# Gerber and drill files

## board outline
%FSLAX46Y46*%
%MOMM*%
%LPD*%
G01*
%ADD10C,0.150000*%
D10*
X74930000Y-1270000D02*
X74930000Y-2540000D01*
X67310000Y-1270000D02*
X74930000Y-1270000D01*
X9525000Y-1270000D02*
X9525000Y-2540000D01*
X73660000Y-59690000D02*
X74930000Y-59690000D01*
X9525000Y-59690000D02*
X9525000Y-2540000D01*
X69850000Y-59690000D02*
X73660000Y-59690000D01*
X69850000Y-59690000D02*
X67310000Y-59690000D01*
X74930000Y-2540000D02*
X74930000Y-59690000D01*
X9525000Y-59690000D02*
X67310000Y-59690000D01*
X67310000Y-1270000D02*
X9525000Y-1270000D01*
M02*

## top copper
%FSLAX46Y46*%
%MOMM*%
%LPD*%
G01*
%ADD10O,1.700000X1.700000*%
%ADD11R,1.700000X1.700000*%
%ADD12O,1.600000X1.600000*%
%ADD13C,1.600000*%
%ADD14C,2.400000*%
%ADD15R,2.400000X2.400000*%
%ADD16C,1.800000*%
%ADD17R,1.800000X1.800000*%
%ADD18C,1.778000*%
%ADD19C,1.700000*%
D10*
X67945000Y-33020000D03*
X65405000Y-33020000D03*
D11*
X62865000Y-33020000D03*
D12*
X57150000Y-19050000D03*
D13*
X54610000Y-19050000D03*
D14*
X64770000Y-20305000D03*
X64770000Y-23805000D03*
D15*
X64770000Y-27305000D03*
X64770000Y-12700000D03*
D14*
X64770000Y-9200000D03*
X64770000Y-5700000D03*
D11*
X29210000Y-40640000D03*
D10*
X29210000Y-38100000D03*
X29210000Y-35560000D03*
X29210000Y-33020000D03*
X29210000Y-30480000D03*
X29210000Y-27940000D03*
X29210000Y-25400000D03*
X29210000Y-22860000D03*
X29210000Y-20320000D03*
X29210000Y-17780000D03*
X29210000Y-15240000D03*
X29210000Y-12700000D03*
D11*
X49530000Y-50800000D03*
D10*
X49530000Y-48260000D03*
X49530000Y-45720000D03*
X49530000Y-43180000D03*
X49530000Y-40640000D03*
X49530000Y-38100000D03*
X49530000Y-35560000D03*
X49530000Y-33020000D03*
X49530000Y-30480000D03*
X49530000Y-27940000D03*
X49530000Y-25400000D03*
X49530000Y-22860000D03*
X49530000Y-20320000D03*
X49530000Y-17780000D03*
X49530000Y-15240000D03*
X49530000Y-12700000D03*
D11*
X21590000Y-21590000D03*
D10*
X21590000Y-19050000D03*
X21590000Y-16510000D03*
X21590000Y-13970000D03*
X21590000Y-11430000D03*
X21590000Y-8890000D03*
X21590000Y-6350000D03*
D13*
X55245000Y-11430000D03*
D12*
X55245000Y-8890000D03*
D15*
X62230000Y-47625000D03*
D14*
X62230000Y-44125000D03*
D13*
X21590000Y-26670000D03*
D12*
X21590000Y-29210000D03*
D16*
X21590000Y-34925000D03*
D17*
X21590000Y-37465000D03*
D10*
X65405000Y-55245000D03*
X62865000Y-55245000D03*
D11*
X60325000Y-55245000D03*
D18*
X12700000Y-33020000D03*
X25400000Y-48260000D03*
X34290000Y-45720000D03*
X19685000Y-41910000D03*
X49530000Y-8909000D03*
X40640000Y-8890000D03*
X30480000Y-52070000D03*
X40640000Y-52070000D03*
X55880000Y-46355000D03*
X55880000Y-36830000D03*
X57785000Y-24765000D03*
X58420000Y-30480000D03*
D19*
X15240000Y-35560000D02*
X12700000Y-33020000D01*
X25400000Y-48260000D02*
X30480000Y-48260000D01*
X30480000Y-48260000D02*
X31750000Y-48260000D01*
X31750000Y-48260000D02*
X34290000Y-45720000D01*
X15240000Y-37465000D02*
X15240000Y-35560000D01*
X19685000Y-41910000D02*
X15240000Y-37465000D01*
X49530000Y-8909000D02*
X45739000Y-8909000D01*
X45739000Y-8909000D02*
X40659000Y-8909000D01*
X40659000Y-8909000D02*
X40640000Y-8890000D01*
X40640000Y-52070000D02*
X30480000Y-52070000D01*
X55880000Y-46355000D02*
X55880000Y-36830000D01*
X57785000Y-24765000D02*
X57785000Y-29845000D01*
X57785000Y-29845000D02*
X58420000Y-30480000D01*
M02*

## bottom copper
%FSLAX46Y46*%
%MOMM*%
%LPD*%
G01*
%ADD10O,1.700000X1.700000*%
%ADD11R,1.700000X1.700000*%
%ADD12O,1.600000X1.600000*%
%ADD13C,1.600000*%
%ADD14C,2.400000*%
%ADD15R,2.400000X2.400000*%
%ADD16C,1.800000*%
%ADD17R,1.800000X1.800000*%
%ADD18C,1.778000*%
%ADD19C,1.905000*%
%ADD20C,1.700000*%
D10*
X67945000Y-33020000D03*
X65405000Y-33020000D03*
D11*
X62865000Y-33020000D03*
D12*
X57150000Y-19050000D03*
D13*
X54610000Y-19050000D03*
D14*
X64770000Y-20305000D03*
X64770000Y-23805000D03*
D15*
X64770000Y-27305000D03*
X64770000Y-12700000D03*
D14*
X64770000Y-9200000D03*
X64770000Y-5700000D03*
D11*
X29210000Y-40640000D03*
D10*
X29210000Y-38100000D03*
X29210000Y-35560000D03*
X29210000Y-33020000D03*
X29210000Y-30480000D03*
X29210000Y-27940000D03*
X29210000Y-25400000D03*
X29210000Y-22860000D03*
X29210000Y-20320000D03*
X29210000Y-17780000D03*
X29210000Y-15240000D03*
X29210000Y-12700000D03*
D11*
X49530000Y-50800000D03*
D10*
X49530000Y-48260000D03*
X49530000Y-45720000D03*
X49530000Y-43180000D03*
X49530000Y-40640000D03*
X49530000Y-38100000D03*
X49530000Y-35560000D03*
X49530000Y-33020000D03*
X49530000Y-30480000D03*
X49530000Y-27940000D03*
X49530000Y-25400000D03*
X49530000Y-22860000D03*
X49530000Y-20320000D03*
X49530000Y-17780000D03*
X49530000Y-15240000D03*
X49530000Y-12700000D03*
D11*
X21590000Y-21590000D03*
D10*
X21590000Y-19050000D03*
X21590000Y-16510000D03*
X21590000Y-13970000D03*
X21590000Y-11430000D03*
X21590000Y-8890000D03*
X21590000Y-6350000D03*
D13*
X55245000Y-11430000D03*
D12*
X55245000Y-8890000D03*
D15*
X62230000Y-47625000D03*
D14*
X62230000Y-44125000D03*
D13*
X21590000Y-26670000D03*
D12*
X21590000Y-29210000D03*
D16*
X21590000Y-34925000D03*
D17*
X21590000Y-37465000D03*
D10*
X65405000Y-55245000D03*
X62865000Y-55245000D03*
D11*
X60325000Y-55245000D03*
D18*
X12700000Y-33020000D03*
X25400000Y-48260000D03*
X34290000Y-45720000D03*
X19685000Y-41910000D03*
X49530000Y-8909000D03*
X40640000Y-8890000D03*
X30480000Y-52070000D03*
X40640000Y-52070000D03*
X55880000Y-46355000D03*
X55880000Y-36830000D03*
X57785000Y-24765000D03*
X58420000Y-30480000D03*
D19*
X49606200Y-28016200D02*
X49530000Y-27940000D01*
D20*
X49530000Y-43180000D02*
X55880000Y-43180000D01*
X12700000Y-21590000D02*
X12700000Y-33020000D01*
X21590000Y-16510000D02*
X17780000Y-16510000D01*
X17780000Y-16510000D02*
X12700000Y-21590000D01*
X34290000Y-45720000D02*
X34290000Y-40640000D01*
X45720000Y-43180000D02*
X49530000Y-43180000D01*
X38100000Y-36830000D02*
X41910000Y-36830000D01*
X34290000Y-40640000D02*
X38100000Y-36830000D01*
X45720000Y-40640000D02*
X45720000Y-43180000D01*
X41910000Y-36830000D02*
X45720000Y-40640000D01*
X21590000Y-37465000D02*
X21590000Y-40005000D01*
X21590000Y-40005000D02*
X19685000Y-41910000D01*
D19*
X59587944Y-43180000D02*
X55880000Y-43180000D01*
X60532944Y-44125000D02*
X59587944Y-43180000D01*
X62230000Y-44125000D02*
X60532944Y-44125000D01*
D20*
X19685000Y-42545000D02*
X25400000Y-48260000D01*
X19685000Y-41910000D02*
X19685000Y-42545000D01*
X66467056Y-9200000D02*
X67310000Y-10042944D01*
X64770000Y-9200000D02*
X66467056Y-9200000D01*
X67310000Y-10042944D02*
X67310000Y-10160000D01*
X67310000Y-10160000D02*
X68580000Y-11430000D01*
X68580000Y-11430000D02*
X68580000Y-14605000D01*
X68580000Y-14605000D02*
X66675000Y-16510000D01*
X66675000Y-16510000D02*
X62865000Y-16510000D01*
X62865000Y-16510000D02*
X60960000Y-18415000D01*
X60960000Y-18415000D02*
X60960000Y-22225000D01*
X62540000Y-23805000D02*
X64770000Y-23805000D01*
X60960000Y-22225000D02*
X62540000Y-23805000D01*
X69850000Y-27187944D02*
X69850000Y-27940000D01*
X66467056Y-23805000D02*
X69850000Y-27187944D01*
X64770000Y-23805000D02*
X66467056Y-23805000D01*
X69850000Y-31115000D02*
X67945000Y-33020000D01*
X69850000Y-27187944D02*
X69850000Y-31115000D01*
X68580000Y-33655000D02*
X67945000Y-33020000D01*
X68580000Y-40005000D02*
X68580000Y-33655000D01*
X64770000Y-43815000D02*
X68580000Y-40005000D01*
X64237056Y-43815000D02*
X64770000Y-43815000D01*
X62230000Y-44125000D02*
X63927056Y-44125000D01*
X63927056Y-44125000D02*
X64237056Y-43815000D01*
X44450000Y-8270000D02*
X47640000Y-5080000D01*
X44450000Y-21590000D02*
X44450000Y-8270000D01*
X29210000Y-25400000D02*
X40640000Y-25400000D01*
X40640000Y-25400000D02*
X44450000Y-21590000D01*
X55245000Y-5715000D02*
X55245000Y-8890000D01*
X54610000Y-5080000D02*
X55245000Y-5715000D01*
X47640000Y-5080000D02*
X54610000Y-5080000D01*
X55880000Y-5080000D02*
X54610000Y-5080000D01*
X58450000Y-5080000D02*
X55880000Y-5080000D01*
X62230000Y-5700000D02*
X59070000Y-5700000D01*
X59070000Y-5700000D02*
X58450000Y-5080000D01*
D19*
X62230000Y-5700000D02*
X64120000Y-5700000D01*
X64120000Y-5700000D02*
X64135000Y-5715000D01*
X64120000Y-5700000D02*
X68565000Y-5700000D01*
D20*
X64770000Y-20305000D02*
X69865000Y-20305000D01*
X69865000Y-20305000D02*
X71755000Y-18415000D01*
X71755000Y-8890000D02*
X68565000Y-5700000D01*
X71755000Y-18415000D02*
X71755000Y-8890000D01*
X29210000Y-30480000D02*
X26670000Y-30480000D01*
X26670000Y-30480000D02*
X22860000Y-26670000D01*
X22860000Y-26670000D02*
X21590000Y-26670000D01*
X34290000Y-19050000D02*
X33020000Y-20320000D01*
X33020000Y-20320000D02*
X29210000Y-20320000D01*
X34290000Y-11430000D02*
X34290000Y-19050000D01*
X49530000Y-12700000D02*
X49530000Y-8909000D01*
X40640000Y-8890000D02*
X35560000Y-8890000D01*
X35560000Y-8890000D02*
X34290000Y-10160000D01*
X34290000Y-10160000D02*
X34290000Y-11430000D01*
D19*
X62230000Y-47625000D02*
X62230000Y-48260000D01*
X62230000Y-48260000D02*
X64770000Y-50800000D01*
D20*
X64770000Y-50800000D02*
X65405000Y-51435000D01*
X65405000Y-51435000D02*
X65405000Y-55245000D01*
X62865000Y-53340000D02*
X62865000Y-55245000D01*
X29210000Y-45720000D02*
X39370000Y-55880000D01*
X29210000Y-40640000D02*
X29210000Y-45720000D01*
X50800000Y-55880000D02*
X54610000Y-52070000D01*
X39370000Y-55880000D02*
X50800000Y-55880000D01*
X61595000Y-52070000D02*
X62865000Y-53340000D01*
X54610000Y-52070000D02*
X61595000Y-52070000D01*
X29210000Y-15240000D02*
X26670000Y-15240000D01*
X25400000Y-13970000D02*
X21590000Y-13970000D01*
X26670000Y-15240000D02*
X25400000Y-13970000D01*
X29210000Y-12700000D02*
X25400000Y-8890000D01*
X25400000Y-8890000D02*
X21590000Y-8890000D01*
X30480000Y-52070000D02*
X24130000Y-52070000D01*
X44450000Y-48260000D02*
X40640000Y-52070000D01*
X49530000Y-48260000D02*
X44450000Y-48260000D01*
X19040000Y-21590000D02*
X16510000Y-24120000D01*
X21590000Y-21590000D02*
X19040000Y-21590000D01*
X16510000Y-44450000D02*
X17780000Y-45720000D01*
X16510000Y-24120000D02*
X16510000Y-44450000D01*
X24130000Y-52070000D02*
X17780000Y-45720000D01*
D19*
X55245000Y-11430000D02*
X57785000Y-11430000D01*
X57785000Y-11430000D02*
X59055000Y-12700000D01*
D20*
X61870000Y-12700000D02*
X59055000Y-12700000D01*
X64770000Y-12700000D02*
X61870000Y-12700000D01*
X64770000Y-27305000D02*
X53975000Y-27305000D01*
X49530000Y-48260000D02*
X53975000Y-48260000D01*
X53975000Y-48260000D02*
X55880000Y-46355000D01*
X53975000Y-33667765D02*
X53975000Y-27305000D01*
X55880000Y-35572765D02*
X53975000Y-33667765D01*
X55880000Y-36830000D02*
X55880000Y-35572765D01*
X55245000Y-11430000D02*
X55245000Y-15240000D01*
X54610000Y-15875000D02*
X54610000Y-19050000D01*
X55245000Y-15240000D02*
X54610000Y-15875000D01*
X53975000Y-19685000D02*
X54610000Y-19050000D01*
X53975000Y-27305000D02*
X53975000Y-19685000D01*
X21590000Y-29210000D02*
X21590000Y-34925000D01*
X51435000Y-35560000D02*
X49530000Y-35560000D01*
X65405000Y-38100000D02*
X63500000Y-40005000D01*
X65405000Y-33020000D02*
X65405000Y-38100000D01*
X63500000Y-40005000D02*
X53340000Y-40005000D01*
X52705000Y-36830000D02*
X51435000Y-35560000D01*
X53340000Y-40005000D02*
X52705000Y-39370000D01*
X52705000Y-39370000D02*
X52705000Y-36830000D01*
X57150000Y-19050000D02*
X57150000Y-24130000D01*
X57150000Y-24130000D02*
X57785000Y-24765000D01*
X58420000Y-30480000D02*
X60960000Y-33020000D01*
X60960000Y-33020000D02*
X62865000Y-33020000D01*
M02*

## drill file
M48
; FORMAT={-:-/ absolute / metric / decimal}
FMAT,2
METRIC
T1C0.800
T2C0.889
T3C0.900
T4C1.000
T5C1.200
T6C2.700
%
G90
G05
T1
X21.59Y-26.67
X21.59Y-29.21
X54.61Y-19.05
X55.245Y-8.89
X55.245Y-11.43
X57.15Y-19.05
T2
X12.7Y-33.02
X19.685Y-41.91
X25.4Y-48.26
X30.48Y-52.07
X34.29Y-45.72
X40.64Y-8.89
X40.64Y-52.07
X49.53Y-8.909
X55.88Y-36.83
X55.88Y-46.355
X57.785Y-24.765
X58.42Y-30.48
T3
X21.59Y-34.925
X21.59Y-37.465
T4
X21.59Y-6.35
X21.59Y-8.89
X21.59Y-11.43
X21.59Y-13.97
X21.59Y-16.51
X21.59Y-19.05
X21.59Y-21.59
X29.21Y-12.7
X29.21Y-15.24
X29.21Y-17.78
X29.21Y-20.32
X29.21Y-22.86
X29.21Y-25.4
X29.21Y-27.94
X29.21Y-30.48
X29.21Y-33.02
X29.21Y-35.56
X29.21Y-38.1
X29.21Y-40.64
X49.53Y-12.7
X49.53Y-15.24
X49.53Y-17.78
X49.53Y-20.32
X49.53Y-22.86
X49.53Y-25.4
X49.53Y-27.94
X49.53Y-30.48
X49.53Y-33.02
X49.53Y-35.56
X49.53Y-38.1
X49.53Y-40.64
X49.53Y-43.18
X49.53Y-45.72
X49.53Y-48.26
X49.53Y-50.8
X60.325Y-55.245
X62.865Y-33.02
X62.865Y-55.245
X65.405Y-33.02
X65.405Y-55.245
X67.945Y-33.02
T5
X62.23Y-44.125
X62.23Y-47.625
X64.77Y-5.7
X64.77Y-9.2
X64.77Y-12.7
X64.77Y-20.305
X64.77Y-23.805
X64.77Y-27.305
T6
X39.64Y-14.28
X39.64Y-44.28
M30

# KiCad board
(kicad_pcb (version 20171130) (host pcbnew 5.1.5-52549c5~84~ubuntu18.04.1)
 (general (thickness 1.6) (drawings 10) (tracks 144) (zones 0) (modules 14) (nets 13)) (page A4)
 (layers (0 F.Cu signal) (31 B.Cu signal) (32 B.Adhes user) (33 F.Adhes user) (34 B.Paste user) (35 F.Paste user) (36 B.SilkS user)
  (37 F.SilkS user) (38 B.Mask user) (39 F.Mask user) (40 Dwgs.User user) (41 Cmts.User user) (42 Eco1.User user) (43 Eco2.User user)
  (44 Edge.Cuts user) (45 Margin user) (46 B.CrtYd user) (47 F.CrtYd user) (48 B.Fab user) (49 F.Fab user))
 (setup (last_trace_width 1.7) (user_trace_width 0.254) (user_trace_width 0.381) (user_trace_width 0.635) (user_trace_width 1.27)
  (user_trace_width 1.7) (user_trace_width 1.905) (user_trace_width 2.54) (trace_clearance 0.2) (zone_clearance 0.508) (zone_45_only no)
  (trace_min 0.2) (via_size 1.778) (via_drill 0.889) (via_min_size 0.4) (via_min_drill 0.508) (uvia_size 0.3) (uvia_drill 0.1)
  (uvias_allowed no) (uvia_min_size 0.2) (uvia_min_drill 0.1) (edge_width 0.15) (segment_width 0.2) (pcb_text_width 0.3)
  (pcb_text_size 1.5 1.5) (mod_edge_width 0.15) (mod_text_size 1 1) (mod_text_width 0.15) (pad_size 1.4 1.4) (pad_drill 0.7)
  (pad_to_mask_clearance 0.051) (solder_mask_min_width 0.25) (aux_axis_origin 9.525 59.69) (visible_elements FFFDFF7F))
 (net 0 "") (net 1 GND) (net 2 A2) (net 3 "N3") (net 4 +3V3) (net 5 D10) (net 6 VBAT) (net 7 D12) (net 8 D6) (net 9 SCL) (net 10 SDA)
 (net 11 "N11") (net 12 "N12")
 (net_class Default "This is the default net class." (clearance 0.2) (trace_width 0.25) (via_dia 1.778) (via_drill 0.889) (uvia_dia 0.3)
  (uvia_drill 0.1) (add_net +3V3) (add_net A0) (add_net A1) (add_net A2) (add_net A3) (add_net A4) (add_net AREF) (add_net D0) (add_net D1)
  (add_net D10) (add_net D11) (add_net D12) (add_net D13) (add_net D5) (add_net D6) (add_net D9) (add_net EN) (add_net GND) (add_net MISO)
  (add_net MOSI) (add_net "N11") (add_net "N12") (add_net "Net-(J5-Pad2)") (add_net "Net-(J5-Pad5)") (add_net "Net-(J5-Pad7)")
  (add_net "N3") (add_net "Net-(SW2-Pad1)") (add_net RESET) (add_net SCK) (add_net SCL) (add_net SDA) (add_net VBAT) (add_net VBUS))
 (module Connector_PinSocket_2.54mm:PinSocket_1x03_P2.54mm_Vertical (layer F.Cu) (at 62.865 33.02 90)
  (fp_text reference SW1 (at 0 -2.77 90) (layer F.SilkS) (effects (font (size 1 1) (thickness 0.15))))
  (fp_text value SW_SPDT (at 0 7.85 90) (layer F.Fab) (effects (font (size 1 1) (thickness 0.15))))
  (pad 3 thru_hole oval (at 0 5.08 90) (size 1.7 1.7) (drill 1) (layers *.Cu *.Mask) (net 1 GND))
  (pad 2 thru_hole oval (at 0 2.54 90) (size 1.7 1.7) (drill 1) (layers *.Cu *.Mask) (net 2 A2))
  (pad 1 thru_hole rect (at 0 0 90) (size 1.7 1.7) (drill 1) (layers *.Cu *.Mask) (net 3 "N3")))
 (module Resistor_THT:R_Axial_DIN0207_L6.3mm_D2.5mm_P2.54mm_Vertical (layer F.Cu) (at 54.61 19.05)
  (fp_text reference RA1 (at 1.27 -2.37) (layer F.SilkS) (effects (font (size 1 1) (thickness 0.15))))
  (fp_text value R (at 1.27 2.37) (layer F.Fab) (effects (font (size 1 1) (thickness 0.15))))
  (pad 2 thru_hole oval (at 2.54 0) (size 1.6 1.6) (drill 0.8) (layers *.Cu *.Mask) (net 3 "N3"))
  (pad 1 thru_hole circle (at 0 0) (size 1.6 1.6) (drill 0.8) (layers *.Cu *.Mask) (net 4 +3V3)))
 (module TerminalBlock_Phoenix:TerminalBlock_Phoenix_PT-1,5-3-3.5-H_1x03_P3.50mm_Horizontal (layer F.Cu) (at 64.77 27.305 90)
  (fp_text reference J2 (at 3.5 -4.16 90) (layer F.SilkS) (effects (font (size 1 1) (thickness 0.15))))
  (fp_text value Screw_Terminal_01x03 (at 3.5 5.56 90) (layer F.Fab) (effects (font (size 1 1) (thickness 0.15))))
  (pad 3 thru_hole circle (at 7 0 90) (size 2.4 2.4) (drill 1.2) (layers *.Cu *.Mask) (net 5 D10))
  (pad 2 thru_hole circle (at 3.5 0 90) (size 2.4 2.4) (drill 1.2) (layers *.Cu *.Mask) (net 1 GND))
  (pad 1 thru_hole rect (at 0 0 90) (size 2.4 2.4) (drill 1.2) (layers *.Cu *.Mask) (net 4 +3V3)))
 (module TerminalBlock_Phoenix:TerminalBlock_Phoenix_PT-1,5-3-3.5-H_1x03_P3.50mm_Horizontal (layer F.Cu) (at 64.77 12.7 90)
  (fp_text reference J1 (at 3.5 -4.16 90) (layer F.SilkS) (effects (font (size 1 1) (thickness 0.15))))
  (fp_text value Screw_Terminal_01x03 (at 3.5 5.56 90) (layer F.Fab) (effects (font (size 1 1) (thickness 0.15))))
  (pad 1 thru_hole rect (at 0 0 90) (size 2.4 2.4) (drill 1.2) (layers *.Cu *.Mask) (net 4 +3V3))
  (pad 2 thru_hole circle (at 3.5 0 90) (size 2.4 2.4) (drill 1.2) (layers *.Cu *.Mask) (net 1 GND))
  (pad 3 thru_hole circle (at 7 0 90) (size 2.4 2.4) (drill 1.2) (layers *.Cu *.Mask) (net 5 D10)))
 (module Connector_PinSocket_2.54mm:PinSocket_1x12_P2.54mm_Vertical (layer F.Cu) (at 29.21 40.64 180)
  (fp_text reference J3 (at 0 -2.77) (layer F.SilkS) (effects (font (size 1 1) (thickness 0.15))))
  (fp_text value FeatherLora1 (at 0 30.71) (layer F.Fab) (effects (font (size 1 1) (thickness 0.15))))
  (pad 1 thru_hole rect (at 0 0 180) (size 1.7 1.7) (drill 1) (layers *.Cu *.Mask) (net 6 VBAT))
  (pad 2 thru_hole oval (at 0 2.54 180) (size 1.7 1.7) (drill 1) (layers *.Cu *.Mask))
  (pad 3 thru_hole oval (at 0 5.08 180) (size 1.7 1.7) (drill 1) (layers *.Cu *.Mask))
  (pad 4 thru_hole oval (at 0 7.62 180) (size 1.7 1.7) (drill 1) (layers *.Cu *.Mask))
  (pad 5 thru_hole oval (at 0 10.16 180) (size 1.7 1.7) (drill 1) (layers *.Cu *.Mask) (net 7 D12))
  (pad 6 thru_hole oval (at 0 12.7 180) (size 1.7 1.7) (drill 1) (layers *.Cu *.Mask))
  (pad 7 thru_hole oval (at 0 15.24 180) (size 1.7 1.7) (drill 1) (layers *.Cu *.Mask) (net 5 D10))
  (pad 8 thru_hole oval (at 0 17.78 180) (size 1.7 1.7) (drill 1) (layers *.Cu *.Mask))
  (pad 9 thru_hole oval (at 0 20.32 180) (size 1.7 1.7) (drill 1) (layers *.Cu *.Mask) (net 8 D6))
  (pad 10 thru_hole oval (at 0 22.86 180) (size 1.7 1.7) (drill 1) (layers *.Cu *.Mask))
  (pad 11 thru_hole oval (at 0 25.4 180) (size 1.7 1.7) (drill 1) (layers *.Cu *.Mask) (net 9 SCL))
  (pad 12 thru_hole oval (at 0 27.94 180) (size 1.7 1.7) (drill 1) (layers *.Cu *.Mask) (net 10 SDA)))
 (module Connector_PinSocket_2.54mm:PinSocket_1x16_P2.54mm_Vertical (layer F.Cu) (at 49.53 50.8 180)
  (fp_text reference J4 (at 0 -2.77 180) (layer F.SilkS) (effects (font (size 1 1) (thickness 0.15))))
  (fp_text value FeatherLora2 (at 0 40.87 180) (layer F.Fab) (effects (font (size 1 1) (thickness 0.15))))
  (pad 1 thru_hole rect (at 0 0 180) (size 1.7 1.7) (drill 1) (layers *.Cu *.Mask))
  (pad 2 thru_hole oval (at 0 2.54 180) (size 1.7 1.7) (drill 1) (layers *.Cu *.Mask) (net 4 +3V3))
  (pad 3 thru_hole oval (at 0 5.08 180) (size 1.7 1.7) (drill 1) (layers *.Cu *.Mask))
  (pad 4 thru_hole oval (at 0 7.62 180) (size 1.7 1.7) (drill 1) (layers *.Cu *.Mask) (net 1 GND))
  (pad 5 thru_hole oval (at 0 10.16 180) (size 1.7 1.7) (drill 1) (layers *.Cu *.Mask))
  (pad 6 thru_hole oval (at 0 12.7 180) (size 1.7 1.7) (drill 1) (layers *.Cu *.Mask))
  (pad 7 thru_hole oval (at 0 15.24 180) (size 1.7 1.7) (drill 1) (layers *.Cu *.Mask) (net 2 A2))
  (pad 8 thru_hole oval (at 0 17.78 180) (size 1.7 1.7) (drill 1) (layers *.Cu *.Mask))
  (pad 9 thru_hole oval (at 0 20.32 180) (size 1.7 1.7) (drill 1) (layers *.Cu *.Mask))
  (pad 10 thru_hole oval (at 0 22.86 180) (size 1.7 1.7) (drill 1) (layers *.Cu *.Mask))
  (pad 11 thru_hole oval (at 0 25.4 180) (size 1.7 1.7) (drill 1) (layers *.Cu *.Mask))
  (pad 12 thru_hole oval (at 0 27.94 180) (size 1.7 1.7) (drill 1) (layers *.Cu *.Mask))
  (pad 13 thru_hole oval (at 0 30.48 180) (size 1.7 1.7) (drill 1) (layers *.Cu *.Mask))
  (pad 14 thru_hole oval (at 0 33.02 180) (size 1.7 1.7) (drill 1) (layers *.Cu *.Mask))
  (pad 15 thru_hole oval (at 0 35.56 180) (size 1.7 1.7) (drill 1) (layers *.Cu *.Mask))
  (pad 16 thru_hole oval (at 0 38.1 180) (size 1.7 1.7) (drill 1) (layers *.Cu *.Mask) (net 8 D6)))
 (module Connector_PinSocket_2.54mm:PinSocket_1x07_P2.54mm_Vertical (layer F.Cu) (at 21.59 21.59 180)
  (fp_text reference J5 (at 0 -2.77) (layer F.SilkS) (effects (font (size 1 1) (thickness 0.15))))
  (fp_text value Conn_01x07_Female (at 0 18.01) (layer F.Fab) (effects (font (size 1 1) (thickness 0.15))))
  (pad 1 thru_hole rect (at 0 0 180) (size 1.7 1.7) (drill 1) (layers *.Cu *.Mask) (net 4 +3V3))
  (pad 2 thru_hole oval (at 0 2.54 180) (size 1.7 1.7) (drill 1) (layers *.Cu *.Mask))
  (pad 3 thru_hole oval (at 0 5.08 180) (size 1.7 1.7) (drill 1) (layers *.Cu *.Mask) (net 1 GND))
  (pad 4 thru_hole oval (at 0 7.62 180) (size 1.7 1.7) (drill 1) (layers *.Cu *.Mask) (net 9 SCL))
  (pad 5 thru_hole oval (at 0 10.16 180) (size 1.7 1.7) (drill 1) (layers *.Cu *.Mask))
  (pad 6 thru_hole oval (at 0 12.7 180) (size 1.7 1.7) (drill 1) (layers *.Cu *.Mask) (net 10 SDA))
  (pad 7 thru_hole oval (at 0 15.24 180) (size 1.7 1.7) (drill 1) (layers *.Cu *.Mask)))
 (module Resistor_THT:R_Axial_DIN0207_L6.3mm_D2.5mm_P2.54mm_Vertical (layer F.Cu) (at 55.245 11.43 90)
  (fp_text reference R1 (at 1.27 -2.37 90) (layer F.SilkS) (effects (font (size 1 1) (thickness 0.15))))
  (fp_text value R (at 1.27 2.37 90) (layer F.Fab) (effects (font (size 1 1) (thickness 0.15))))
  (pad 1 thru_hole circle (at 0 0 90) (size 1.6 1.6) (drill 0.8) (layers *.Cu *.Mask) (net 4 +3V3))
  (pad 2 thru_hole oval (at 2.54 0 90) (size 1.6 1.6) (drill 0.8) (layers *.Cu *.Mask) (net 5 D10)))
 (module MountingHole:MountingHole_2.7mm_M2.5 (layer F.Cu) (at 39.64 44.28)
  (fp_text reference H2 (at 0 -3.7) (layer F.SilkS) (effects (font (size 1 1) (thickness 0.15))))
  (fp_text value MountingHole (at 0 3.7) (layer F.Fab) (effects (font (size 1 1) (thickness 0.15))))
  (pad 1 np_thru_hole circle (at 0 0) (size 2.7 2.7) (drill 2.7) (layers *.Cu *.Mask)))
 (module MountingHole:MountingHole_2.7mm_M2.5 (layer F.Cu) (at 39.64 14.28)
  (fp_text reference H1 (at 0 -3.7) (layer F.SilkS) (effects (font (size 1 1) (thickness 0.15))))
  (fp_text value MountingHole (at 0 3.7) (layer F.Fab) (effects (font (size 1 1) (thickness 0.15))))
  (pad 1 np_thru_hole circle (at 0 0) (size 2.7 2.7) (drill 2.7) (layers *.Cu *.Mask)))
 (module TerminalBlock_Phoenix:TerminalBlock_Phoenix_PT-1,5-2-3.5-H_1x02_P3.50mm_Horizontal (layer F.Cu) (at 62.23 47.625 90)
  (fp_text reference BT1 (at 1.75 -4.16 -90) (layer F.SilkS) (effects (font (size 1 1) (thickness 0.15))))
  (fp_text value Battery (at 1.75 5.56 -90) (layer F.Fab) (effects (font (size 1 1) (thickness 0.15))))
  (pad 1 thru_hole rect (at 0 0 90) (size 2.4 2.4) (drill 1.2) (layers *.Cu *.Mask) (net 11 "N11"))
  (pad 2 thru_hole circle (at 3.5 0 90) (size 2.4 2.4) (drill 1.2) (layers *.Cu *.Mask) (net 1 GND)))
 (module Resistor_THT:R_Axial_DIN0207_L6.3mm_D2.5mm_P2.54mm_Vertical (layer F.Cu) (at 21.59 26.67 270)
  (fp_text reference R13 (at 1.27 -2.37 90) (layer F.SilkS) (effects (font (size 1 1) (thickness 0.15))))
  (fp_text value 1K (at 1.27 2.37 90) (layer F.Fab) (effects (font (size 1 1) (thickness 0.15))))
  (pad 1 thru_hole circle (at 0 0 270) (size 1.6 1.6) (drill 0.8) (layers *.Cu *.Mask) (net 7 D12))
  (pad 2 thru_hole oval (at 2.54 0 270) (size 1.6 1.6) (drill 0.8) (layers *.Cu *.Mask) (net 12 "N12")))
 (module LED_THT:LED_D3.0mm (layer F.Cu) (at 21.59 37.465 90)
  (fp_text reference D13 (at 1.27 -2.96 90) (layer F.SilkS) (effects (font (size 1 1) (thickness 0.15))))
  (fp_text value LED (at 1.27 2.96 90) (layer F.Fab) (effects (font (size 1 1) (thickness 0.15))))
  (pad 2 thru_hole circle (at 2.54 0 90) (size 1.8 1.8) (drill 0.9) (layers *.Cu *.Mask) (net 12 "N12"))
  (pad 1 thru_hole rect (at 0 0 90) (size 1.8 1.8) (drill 0.9) (layers *.Cu *.Mask) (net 1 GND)))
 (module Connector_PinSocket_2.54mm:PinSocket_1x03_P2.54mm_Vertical (layer F.Cu) (at 60.325 55.245 90)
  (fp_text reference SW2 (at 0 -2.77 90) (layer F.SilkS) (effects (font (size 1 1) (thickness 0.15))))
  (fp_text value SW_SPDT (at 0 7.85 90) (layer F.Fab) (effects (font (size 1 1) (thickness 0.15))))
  (pad 3 thru_hole oval (at 0 5.08 90) (size 1.7 1.7) (drill 1) (layers *.Cu *.Mask) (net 11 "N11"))
  (pad 2 thru_hole oval (at 0 2.54 90) (size 1.7 1.7) (drill 1) (layers *.Cu *.Mask) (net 6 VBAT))
  (pad 1 thru_hole rect (at 0 0 90) (size 1.7 1.7) (drill 1) (layers *.Cu *.Mask)))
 (gr_line (start 74.93 1.27) (end 74.93 2.54) (layer Edge.Cuts) (width 0.15))
 (gr_line (start 67.31 1.27) (end 74.93 1.27) (layer Edge.Cuts) (width 0.15))
 (gr_line (start 9.525 1.27) (end 9.525 2.54) (layer Edge.Cuts) (width 0.15))
 (gr_line (start 73.66 59.69) (end 74.93 59.69) (layer Edge.Cuts) (width 0.15))
 (gr_line (start 9.525 59.69) (end 9.525 2.54) (layer Edge.Cuts) (width 0.15))
 (gr_line (start 69.85 59.69) (end 73.66 59.69) (layer Edge.Cuts) (width 0.15))
 (gr_line (start 69.85 59.69) (end 67.31 59.69) (layer Edge.Cuts) (width 0.15))
 (gr_line (start 74.93 2.54) (end 74.93 59.69) (layer Edge.Cuts) (width 0.15))
 (gr_line (start 9.525 59.69) (end 67.31 59.69) (layer Edge.Cuts) (width 0.15))
 (gr_line (start 67.31 1.27) (end 9.525 1.27) (layer Edge.Cuts) (width 0.15))
 (segment (start 49.6062 28.0162) (end 49.53 27.94) (width 1.905) (layer B.Cu) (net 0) (status 30))
 (segment (start 49.53 43.18) (end 55.88 43.18) (width 1.7) (layer B.Cu) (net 1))
 (via (at 12.7 33.02) (size 1.778) (drill 0.889) (layers F.Cu B.Cu) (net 1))
 (segment (start 15.24 35.56) (end 12.7 33.02) (width 1.7) (layer F.Cu) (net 1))
 (segment (start 12.7 21.59) (end 12.7 33.02) (width 1.7) (layer B.Cu) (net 1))
 (segment (start 21.59 16.51) (end 17.78 16.51) (width 1.7) (layer B.Cu) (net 1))
 (segment (start 17.78 16.51) (end 12.7 21.59) (width 1.7) (layer B.Cu) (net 1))
 (segment (start 25.4 48.26) (end 30.48 48.26) (width 1.7) (layer F.Cu) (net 1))
 (segment (start 30.48 48.26) (end 31.75 48.26) (width 1.7) (layer F.Cu) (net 1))
 (via (at 25.4 48.26) (size 1.778) (drill 0.889) (layers F.Cu B.Cu) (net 1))
 (segment (start 34.29 45.72) (end 34.29 40.64) (width 1.7) (layer B.Cu) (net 1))
 (segment (start 31.75 48.26) (end 34.29 45.72) (width 1.7) (layer F.Cu) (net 1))
 (segment (start 45.72 43.18) (end 49.53 43.18) (width 1.7) (layer B.Cu) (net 1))
 (segment (start 38.1 36.83) (end 41.91 36.83) (width 1.7) (layer B.Cu) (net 1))
 (segment (start 34.29 40.64) (end 38.1 36.83) (width 1.7) (layer B.Cu) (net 1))
 (segment (start 45.72 40.64) (end 45.72 43.18) (width 1.7) (layer B.Cu) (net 1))
 (segment (start 41.91 36.83) (end 45.72 40.64) (width 1.7) (layer B.Cu) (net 1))
 (via (at 34.29 45.72) (size 1.778) (drill 0.889) (layers F.Cu B.Cu) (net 1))
 (segment (start 21.59 37.465) (end 21.59 40.005) (width 1.7) (layer B.Cu) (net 1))
 (via (at 19.685 41.91) (size 1.778) (drill 0.889) (layers F.Cu B.Cu) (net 1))
 (segment (start 21.59 40.005) (end 19.685 41.91) (width 1.7) (layer B.Cu) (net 1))
 (segment (start 15.24 37.465) (end 15.24 35.56) (width 1.7) (layer F.Cu) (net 1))
 (segment (start 19.685 41.91) (end 15.24 37.465) (width 1.7) (layer F.Cu) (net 1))
 (segment (start 59.587944 43.18) (end 55.88 43.18) (width 1.905) (layer B.Cu) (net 1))
 (segment (start 60.532944 44.125) (end 59.587944 43.18) (width 1.905) (layer B.Cu) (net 1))
 (segment (start 62.23 44.125) (end 60.532944 44.125) (width 1.905) (layer B.Cu) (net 1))
 (segment (start 19.685 42.545) (end 25.4 48.26) (width 1.7) (layer B.Cu) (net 1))
 (segment (start 19.685 41.91) (end 19.685 42.545) (width 1.7) (layer B.Cu) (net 1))
 (segment (start 66.467056 9.2) (end 67.31 10.042944) (width 1.7) (layer B.Cu) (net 1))
 (segment (start 64.77 9.2) (end 66.467056 9.2) (width 1.7) (layer B.Cu) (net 1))
 (segment (start 67.31 10.042944) (end 67.31 10.16) (width 1.7) (layer B.Cu) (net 1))
 (segment (start 67.31 10.16) (end 68.58 11.43) (width 1.7) (layer B.Cu) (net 1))
 (segment (start 68.58 11.43) (end 68.58 14.605) (width 1.7) (layer B.Cu) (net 1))
 (segment (start 68.58 14.605) (end 66.675 16.51) (width 1.7) (layer B.Cu) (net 1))
 (segment (start 66.675 16.51) (end 62.865 16.51) (width 1.7) (layer B.Cu) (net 1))
 (segment (start 62.865 16.51) (end 60.96 18.415) (width 1.7) (layer B.Cu) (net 1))
 (segment (start 60.96 18.415) (end 60.96 22.225) (width 1.7) (layer B.Cu) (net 1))
 (segment (start 62.54 23.805) (end 64.77 23.805) (width 1.7) (layer B.Cu) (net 1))
 (segment (start 60.96 22.225) (end 62.54 23.805) (width 1.7) (layer B.Cu) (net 1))
 (segment (start 69.85 27.187944) (end 69.85 27.94) (width 1.7) (layer B.Cu) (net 1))
 (segment (start 66.467056 23.805) (end 69.85 27.187944) (width 1.7) (layer B.Cu) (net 1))
 (segment (start 64.77 23.805) (end 66.467056 23.805) (width 1.7) (layer B.Cu) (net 1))
 (segment (start 69.85 31.115) (end 67.945 33.02) (width 1.7) (layer B.Cu) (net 1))
 (segment (start 69.85 27.187944) (end 69.85 31.115) (width 1.7) (layer B.Cu) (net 1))
 (segment (start 68.58 33.655) (end 67.945 33.02) (width 1.7) (layer B.Cu) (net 1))
 (segment (start 68.58 40.005) (end 68.58 33.655) (width 1.7) (layer B.Cu) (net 1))
 (segment (start 64.77 43.815) (end 68.58 40.005) (width 1.7) (layer B.Cu) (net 1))
 (segment (start 64.237056 43.815) (end 64.77 43.815) (width 1.7) (layer B.Cu) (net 1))
 (segment (start 62.23 44.125) (end 63.927056 44.125) (width 1.7) (layer B.Cu) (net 1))
 (segment (start 63.927056 44.125) (end 64.237056 43.815) (width 1.7) (layer B.Cu) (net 1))
 (segment (start 44.45 8.27) (end 47.64 5.08) (width 1.7) (layer B.Cu) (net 5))
 (segment (start 44.45 21.59) (end 44.45 8.27) (width 1.7) (layer B.Cu) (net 5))
 (segment (start 29.21 25.4) (end 40.64 25.4) (width 1.7) (layer B.Cu) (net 5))
 (segment (start 40.64 25.4) (end 44.45 21.59) (width 1.7) (layer B.Cu) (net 5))
 (segment (start 55.245 5.715) (end 55.245 8.89) (width 1.7) (layer B.Cu) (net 5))
 (segment (start 54.61 5.08) (end 55.245 5.715) (width 1.7) (layer B.Cu) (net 5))
 (segment (start 47.64 5.08) (end 54.61 5.08) (width 1.7) (layer B.Cu) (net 5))
 (segment (start 55.88 5.08) (end 54.61 5.08) (width 1.7) (layer B.Cu) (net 5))
 (segment (start 58.45 5.08) (end 55.88 5.08) (width 1.7) (layer B.Cu) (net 5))
 (segment (start 62.23 5.7) (end 59.07 5.7) (width 1.7) (layer B.Cu) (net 5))
 (segment (start 59.07 5.7) (end 58.45 5.08) (width 1.7) (layer B.Cu) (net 5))
 (segment (start 62.23 5.7) (end 64.12 5.7) (width 1.905) (layer B.Cu) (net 5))
 (segment (start 64.12 5.7) (end 64.135 5.715) (width 1.905) (layer B.Cu) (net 5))
 (segment (start 64.12 5.7) (end 68.565 5.7) (width 1.905) (layer B.Cu) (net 5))
 (segment (start 64.77 20.305) (end 69.865 20.305) (width 1.7) (layer B.Cu) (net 5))
 (segment (start 69.865 20.305) (end 71.755 18.415) (width 1.7) (layer B.Cu) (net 5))
 (segment (start 71.755 8.89) (end 68.565 5.7) (width 1.7) (layer B.Cu) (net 5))
 (segment (start 71.755 18.415) (end 71.755 8.89) (width 1.7) (layer B.Cu) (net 5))
 (segment (start 29.21 30.48) (end 26.67 30.48) (width 1.7) (layer B.Cu) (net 7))
 (segment (start 26.67 30.48) (end 22.86 26.67) (width 1.7) (layer B.Cu) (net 7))
 (segment (start 22.86 26.67) (end 21.59 26.67) (width 1.7) (layer B.Cu) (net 7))
 (segment (start 34.29 19.05) (end 33.02 20.32) (width 1.7) (layer B.Cu) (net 8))
 (via (at 49.53 8.909) (size 1.778) (drill 0.889) (layers F.Cu B.Cu) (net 8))
 (segment (start 33.02 20.32) (end 29.21 20.32) (width 1.7) (layer B.Cu) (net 8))
 (segment (start 34.29 11.43) (end 34.29 19.05) (width 1.7) (layer B.Cu) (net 8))
 (segment (start 49.53 12.7) (end 49.53 8.909) (width 1.7) (layer B.Cu) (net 8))
 (segment (start 49.53 8.909) (end 45.739 8.909) (width 1.7) (layer F.Cu) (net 8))
 (via (at 40.64 8.89) (size 1.778) (drill 0.889) (layers F.Cu B.Cu) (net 8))
 (segment (start 45.739 8.909) (end 40.659 8.909) (width 1.7) (layer F.Cu) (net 8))
 (segment (start 40.659 8.909) (end 40.64 8.89) (width 1.7) (layer F.Cu) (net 8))
 (segment (start 40.64 8.89) (end 35.56 8.89) (width 1.7) (layer B.Cu) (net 8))
 (segment (start 35.56 8.89) (end 34.29 10.16) (width 1.7) (layer B.Cu) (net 8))
 (segment (start 34.29 10.16) (end 34.29 11.43) (width 1.7) (layer B.Cu) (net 8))
 (segment (start 62.23 47.625) (end 62.23 48.26) (width 1.905) (layer B.Cu) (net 11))
 (segment (start 62.23 48.26) (end 64.77 50.8) (width 1.905) (layer B.Cu) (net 11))
 (segment (start 64.77 50.8) (end 65.405 51.435) (width 1.7) (layer B.Cu) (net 11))
 (segment (start 65.405 51.435) (end 65.405 55.245) (width 1.7) (layer B.Cu) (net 11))
 (segment (start 62.865 53.34) (end 62.865 55.245) (width 1.7) (layer B.Cu) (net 6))
 (segment (start 29.21 45.72) (end 39.37 55.88) (width 1.7) (layer B.Cu) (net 6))
 (segment (start 29.21 40.64) (end 29.21 45.72) (width 1.7) (layer B.Cu) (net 6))
 (segment (start 50.8 55.88) (end 54.61 52.07) (width 1.7) (layer B.Cu) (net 6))
 (segment (start 39.37 55.88) (end 50.8 55.88) (width 1.7) (layer B.Cu) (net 6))
 (segment (start 61.595 52.07) (end 62.865 53.34) (width 1.7) (layer B.Cu) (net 6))
 (segment (start 54.61 52.07) (end 61.595 52.07) (width 1.7) (layer B.Cu) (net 6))
 (segment (start 29.21 15.24) (end 26.67 15.24) (width 1.7) (layer B.Cu) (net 9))
 (segment (start 25.4 13.97) (end 21.59 13.97) (width 1.7) (layer B.Cu) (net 9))
 (segment (start 26.67 15.24) (end 25.4 13.97) (width 1.7) (layer B.Cu) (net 9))
 (segment (start 29.21 12.7) (end 25.4 8.89) (width 1.7) (layer B.Cu) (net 10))
 (segment (start 25.4 8.89) (end 21.59 8.89) (width 1.7) (layer B.Cu) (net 10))
 (segment (start 30.48 52.07) (end 24.13 52.07) (width 1.7) (layer B.Cu) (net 4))
 (segment (start 44.45 48.26) (end 40.64 52.07) (width 1.7) (layer B.Cu) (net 4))
 (segment (start 49.53 48.26) (end 44.45 48.26) (width 1.7) (layer B.Cu) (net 4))
 (via (at 30.48 52.07) (size 1.778) (drill 0.889) (layers F.Cu B.Cu) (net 4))
 (via (at 40.64 52.07) (size 1.778) (drill 0.889) (layers F.Cu B.Cu) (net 4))
 (segment (start 40.64 52.07) (end 30.48 52.07) (width 1.7) (layer F.Cu) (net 4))
 (segment (start 19.04 21.59) (end 16.51 24.12) (width 1.7) (layer B.Cu) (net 4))
 (segment (start 21.59 21.59) (end 19.04 21.59) (width 1.7) (layer B.Cu) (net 4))
 (segment (start 16.51 44.45) (end 17.78 45.72) (width 1.7) (layer B.Cu) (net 4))
 (segment (start 16.51 24.12) (end 16.51 44.45) (width 1.7) (layer B.Cu) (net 4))
 (segment (start 24.13 52.07) (end 17.78 45.72) (width 1.7) (layer B.Cu) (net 4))
 (segment (start 55.245 11.43) (end 57.785 11.43) (width 1.905) (layer B.Cu) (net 4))
 (segment (start 57.785 11.43) (end 59.055 12.7) (width 1.905) (layer B.Cu) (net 4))
 (segment (start 61.87 12.7) (end 59.055 12.7) (width 1.7) (layer B.Cu) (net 4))
 (segment (start 64.77 12.7) (end 61.87 12.7) (width 1.7) (layer B.Cu) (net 4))
 (segment (start 64.77 27.305) (end 53.975 27.305) (width 1.7) (layer B.Cu) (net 4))
 (via (at 55.88 46.355) (size 1.778) (drill 0.889) (layers F.Cu B.Cu) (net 4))
 (segment (start 49.53 48.26) (end 53.975 48.26) (width 1.7) (layer B.Cu) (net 4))
 (segment (start 53.975 48.26) (end 55.88 46.355) (width 1.7) (layer B.Cu) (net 4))
 (via (at 55.88 36.83) (size 1.778) (drill 0.889) (layers F.Cu B.Cu) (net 4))
 (segment (start 55.88 46.355) (end 55.88 36.83) (width 1.7) (layer F.Cu) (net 4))
 (segment (start 53.975 33.667765) (end 53.975 27.305) (width 1.7) (layer B.Cu) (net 4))
 (segment (start 55.88 35.572765) (end 53.975 33.667765) (width 1.7) (layer B.Cu) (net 4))
 (segment (start 55.88 36.83) (end 55.88 35.572765) (width 1.7) (layer B.Cu) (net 4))
 (segment (start 55.245 11.43) (end 55.245 15.24) (width 1.7) (layer B.Cu) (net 4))
 (segment (start 54.61 15.875) (end 54.61 19.05) (width 1.7) (layer B.Cu) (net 4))
 (segment (start 55.245 15.24) (end 54.61 15.875) (width 1.7) (layer B.Cu) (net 4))
 (segment (start 53.975 19.685) (end 54.61 19.05) (width 1.7) (layer B.Cu) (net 4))
 (segment (start 53.975 27.305) (end 53.975 19.685) (width 1.7) (layer B.Cu) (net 4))
 (segment (start 21.59 29.21) (end 21.59 34.925) (width 1.7) (layer B.Cu) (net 12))
 (segment (start 51.435 35.56) (end 49.53 35.56) (width 1.7) (layer B.Cu) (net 2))
 (segment (start 65.405 38.1) (end 63.5 40.005) (width 1.7) (layer B.Cu) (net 2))
 (segment (start 65.405 33.02) (end 65.405 38.1) (width 1.7) (layer B.Cu) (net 2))
 (segment (start 63.5 40.005) (end 53.34 40.005) (width 1.7) (layer B.Cu) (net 2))
 (segment (start 52.705 36.83) (end 51.435 35.56) (width 1.7) (layer B.Cu) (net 2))
 (segment (start 53.34 40.005) (end 52.705 39.37) (width 1.7) (layer B.Cu) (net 2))
 (segment (start 52.705 39.37) (end 52.705 36.83) (width 1.7) (layer B.Cu) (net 2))
 (segment (start 57.15 19.05) (end 57.15 24.13) (width 1.7) (layer B.Cu) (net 3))
 (via (at 57.785 24.765) (size 1.778) (drill 0.889) (layers F.Cu B.Cu) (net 3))
 (segment (start 57.15 24.13) (end 57.785 24.765) (width 1.7) (layer B.Cu) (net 3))
 (via (at 58.42 30.48) (size 1.778) (drill 0.889) (layers F.Cu B.Cu) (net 3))
 (segment (start 57.785 24.765) (end 57.785 29.845) (width 1.7) (layer F.Cu) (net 3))
 (segment (start 57.785 29.845) (end 58.42 30.48) (width 1.7) (layer F.Cu) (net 3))
 (segment (start 58.42 30.48) (end 60.96 33.02) (width 1.7) (layer B.Cu) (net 3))
 (segment (start 60.96 33.02) (end 62.865 33.02) (width 1.7) (layer B.Cu) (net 3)))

